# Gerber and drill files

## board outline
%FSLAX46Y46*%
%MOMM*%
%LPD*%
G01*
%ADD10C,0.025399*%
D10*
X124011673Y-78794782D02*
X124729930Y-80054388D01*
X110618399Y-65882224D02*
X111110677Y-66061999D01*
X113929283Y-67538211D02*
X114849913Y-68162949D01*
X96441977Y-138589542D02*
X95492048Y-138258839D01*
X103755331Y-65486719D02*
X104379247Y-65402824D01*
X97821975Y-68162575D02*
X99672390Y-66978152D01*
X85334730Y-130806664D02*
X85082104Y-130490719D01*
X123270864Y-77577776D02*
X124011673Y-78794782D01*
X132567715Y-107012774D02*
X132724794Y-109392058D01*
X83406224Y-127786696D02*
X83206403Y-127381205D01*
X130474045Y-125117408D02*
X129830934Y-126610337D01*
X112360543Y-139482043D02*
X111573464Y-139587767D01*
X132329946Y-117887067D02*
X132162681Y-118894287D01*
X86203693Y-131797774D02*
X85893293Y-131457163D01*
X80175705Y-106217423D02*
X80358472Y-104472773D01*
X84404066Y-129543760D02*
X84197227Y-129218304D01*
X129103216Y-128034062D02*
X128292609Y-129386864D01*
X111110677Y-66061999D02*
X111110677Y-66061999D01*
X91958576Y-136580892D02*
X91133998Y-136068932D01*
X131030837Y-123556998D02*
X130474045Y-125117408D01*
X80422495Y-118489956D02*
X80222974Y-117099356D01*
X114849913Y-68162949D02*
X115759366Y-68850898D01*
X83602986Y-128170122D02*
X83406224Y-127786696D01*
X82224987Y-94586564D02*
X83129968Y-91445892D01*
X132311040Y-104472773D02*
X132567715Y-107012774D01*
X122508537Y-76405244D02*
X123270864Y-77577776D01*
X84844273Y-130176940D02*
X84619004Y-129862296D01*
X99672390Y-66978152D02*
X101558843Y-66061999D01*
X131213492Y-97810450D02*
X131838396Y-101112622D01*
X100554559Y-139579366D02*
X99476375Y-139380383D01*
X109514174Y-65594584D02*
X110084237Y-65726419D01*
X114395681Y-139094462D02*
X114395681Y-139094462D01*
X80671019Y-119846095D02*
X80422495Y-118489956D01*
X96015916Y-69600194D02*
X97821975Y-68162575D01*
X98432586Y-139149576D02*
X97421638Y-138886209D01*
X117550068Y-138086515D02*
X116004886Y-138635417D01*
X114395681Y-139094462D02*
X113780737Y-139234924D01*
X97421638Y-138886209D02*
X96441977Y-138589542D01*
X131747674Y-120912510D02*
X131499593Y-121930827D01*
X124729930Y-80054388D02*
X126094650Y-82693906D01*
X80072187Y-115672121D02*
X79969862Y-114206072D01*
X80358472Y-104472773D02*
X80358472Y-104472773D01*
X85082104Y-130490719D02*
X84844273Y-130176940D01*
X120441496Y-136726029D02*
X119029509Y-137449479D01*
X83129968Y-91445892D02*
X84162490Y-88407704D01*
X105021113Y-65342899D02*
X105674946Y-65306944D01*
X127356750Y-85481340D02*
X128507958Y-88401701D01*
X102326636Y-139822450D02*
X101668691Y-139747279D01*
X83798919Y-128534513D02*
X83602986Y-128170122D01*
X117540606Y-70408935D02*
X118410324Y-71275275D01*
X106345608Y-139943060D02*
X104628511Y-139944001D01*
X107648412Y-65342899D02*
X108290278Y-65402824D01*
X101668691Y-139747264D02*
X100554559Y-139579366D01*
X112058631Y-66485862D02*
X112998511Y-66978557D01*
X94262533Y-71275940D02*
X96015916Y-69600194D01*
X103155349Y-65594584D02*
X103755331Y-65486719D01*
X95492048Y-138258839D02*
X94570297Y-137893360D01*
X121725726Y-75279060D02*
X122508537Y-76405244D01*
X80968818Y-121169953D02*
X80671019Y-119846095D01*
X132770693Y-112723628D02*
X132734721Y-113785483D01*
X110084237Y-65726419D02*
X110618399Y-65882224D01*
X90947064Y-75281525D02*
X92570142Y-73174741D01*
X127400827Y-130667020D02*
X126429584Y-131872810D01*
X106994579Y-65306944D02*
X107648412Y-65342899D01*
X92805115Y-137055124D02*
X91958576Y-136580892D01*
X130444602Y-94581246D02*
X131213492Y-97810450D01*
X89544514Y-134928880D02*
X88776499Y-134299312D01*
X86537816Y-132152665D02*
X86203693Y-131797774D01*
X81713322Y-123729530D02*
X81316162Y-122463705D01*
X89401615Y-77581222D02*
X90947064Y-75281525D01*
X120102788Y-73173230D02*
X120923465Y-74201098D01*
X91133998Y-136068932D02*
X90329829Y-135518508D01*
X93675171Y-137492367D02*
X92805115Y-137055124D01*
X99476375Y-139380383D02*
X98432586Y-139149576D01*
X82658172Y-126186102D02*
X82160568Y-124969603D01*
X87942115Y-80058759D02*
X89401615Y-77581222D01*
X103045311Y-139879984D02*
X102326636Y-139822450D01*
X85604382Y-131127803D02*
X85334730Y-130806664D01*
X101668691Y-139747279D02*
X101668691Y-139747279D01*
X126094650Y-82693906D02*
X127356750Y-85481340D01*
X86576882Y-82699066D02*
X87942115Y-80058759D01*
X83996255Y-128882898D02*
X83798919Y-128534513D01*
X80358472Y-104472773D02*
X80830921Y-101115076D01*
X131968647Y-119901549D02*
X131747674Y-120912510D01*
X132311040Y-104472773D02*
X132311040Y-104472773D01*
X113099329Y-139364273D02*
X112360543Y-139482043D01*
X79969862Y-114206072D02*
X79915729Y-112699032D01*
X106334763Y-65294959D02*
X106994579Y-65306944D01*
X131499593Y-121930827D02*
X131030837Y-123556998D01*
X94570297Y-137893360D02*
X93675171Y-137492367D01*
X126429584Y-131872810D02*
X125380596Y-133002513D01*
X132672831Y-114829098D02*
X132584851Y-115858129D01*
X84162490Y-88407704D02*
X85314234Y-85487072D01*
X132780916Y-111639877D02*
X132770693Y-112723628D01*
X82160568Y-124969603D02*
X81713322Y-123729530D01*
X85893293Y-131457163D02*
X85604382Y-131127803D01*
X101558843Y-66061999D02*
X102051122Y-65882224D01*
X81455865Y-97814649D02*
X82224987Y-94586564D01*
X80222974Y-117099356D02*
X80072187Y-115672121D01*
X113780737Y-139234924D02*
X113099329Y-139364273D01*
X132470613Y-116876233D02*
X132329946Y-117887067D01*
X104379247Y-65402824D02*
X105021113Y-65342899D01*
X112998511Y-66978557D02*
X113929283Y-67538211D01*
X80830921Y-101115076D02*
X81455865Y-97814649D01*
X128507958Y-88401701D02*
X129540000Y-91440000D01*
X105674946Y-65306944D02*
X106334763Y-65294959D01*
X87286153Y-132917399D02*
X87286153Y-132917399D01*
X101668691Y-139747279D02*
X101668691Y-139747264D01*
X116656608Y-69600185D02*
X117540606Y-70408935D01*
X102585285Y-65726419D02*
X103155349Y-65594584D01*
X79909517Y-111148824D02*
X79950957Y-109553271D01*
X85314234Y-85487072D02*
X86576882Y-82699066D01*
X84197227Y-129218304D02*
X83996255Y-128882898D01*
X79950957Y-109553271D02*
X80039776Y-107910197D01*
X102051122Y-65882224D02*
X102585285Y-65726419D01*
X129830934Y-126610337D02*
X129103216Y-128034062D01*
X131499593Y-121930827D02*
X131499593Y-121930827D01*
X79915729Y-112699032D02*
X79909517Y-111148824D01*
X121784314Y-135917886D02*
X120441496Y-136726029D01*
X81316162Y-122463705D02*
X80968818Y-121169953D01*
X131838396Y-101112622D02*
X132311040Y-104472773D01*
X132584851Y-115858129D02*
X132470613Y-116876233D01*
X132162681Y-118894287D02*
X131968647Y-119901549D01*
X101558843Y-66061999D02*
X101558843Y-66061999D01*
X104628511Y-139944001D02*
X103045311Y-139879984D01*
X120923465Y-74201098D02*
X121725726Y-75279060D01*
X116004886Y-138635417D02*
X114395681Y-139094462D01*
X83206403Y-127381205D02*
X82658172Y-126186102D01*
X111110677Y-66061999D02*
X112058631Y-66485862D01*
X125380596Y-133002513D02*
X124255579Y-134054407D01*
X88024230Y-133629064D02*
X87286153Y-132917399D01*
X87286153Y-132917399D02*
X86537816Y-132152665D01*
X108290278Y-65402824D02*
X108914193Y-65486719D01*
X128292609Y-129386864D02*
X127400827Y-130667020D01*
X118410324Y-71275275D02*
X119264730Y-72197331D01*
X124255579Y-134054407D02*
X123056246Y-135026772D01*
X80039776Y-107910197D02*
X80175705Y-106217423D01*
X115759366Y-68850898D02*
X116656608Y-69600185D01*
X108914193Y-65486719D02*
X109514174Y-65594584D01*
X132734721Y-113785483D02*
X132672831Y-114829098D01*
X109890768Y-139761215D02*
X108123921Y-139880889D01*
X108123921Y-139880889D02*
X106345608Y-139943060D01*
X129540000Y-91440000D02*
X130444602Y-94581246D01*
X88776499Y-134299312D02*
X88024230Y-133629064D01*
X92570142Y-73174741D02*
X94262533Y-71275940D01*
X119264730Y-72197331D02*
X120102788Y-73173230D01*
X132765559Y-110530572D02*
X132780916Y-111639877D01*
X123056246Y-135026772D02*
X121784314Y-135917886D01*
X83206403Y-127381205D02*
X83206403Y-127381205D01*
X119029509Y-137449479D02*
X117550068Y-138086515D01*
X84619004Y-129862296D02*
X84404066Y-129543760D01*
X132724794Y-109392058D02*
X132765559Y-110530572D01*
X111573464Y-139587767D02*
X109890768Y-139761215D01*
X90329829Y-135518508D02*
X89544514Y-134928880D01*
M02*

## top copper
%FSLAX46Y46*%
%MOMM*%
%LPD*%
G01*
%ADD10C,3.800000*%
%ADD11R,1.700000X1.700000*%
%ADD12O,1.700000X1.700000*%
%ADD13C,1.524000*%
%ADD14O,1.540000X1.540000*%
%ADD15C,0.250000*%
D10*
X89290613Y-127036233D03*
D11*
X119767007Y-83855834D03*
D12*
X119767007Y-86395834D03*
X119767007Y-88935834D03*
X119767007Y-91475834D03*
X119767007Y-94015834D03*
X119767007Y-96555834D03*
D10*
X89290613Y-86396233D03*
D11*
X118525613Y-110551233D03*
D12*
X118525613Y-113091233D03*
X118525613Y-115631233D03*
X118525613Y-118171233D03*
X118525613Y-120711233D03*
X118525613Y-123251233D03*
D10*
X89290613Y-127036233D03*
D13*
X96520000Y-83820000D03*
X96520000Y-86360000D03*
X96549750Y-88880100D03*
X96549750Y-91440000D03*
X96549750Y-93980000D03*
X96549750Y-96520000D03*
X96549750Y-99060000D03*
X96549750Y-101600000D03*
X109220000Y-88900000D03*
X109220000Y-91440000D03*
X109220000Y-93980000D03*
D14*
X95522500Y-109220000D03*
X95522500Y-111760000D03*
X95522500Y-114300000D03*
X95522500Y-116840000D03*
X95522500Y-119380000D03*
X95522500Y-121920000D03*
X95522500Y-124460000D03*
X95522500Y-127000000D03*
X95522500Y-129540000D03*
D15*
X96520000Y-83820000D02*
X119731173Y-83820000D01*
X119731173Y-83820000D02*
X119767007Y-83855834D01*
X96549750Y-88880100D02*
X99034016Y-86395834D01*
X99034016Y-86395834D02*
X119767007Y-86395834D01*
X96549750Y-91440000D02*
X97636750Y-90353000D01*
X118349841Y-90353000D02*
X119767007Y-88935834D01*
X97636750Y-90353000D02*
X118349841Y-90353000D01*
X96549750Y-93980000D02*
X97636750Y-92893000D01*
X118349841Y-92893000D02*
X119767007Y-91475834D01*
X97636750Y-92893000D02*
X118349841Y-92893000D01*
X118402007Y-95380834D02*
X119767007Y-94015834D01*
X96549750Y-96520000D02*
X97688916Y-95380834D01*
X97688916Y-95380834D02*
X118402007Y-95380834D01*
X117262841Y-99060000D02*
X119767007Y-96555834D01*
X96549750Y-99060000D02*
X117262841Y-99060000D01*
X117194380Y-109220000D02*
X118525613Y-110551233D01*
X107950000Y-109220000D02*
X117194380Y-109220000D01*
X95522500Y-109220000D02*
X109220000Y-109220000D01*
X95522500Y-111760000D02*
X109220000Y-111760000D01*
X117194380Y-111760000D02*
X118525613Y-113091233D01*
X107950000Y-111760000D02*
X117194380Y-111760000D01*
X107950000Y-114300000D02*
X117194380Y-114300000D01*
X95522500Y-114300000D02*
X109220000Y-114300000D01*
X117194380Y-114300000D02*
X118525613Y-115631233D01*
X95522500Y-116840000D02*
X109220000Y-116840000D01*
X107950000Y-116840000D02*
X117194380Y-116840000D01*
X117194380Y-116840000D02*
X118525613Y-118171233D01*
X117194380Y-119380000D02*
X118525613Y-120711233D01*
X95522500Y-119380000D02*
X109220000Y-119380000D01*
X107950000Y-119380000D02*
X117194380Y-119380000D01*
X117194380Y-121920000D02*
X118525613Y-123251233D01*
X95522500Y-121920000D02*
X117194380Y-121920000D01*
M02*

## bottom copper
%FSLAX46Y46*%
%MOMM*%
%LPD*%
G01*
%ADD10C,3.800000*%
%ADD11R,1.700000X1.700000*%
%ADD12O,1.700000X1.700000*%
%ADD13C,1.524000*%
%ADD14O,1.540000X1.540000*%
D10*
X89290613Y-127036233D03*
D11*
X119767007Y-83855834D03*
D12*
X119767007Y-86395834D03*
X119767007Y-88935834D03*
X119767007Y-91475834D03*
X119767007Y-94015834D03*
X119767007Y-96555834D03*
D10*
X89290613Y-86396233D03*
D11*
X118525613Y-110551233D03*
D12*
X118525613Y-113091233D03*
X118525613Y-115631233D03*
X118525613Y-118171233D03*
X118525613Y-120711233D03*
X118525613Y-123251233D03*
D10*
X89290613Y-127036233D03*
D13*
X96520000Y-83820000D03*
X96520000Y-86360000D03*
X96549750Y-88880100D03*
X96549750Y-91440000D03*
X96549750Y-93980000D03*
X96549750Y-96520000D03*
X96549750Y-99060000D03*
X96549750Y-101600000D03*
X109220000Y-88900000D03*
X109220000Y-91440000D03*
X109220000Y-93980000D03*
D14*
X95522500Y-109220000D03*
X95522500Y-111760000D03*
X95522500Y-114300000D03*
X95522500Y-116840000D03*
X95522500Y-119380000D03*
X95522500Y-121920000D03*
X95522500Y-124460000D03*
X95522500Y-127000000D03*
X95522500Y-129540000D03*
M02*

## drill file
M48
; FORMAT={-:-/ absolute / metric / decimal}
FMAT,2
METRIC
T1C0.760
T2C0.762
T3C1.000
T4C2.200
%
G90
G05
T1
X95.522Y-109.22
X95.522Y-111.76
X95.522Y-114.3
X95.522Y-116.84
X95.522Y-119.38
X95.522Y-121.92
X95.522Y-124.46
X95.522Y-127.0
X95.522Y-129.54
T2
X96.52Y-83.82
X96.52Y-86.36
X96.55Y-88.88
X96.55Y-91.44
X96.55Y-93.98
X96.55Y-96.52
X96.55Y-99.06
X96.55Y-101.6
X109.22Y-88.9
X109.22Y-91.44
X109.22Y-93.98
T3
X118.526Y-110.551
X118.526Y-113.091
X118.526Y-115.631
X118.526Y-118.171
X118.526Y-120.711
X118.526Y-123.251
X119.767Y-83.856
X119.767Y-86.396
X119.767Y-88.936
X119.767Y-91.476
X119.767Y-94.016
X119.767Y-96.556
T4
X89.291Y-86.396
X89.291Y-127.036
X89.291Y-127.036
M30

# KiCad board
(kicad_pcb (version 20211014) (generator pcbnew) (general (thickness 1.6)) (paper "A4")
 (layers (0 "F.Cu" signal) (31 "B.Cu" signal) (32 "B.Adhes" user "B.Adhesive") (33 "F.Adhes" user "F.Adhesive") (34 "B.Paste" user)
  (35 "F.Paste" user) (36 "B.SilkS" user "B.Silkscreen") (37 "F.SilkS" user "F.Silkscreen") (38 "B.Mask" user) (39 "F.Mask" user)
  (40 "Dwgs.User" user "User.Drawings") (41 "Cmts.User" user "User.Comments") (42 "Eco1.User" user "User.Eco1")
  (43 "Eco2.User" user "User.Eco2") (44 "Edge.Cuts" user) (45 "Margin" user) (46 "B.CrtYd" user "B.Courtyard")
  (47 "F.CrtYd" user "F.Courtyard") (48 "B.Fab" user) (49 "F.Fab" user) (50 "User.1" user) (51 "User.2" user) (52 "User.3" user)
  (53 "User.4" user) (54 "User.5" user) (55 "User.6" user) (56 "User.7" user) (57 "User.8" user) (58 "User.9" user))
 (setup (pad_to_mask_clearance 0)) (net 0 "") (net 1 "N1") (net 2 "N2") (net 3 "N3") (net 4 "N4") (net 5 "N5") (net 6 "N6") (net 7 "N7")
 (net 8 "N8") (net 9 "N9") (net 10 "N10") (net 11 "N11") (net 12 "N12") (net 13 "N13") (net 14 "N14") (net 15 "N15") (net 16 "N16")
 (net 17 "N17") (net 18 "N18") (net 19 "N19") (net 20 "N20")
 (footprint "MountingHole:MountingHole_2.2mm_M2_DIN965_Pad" (layer "F.Cu") (at 89.290613 127.036233)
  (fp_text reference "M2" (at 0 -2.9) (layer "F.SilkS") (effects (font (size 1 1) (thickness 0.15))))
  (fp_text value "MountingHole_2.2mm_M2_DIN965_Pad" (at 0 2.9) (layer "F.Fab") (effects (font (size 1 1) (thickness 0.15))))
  (pad "1" thru_hole circle (at 0 0) (size 3.8 3.8) (drill 2.2) (layers *.Cu *.Mask)))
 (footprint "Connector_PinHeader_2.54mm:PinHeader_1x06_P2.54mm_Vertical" (layer "F.Cu") (at 119.767007 83.855834)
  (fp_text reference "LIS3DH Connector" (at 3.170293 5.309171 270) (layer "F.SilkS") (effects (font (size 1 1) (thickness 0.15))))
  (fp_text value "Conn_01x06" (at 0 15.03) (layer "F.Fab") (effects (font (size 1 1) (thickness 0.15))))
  (pad "1" thru_hole rect (at 0 0) (size 1.7 1.7) (drill 1) (layers *.Cu *.Mask) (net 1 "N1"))
  (pad "2" thru_hole oval (at 0 2.54) (size 1.7 1.7) (drill 1) (layers *.Cu *.Mask) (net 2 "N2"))
  (pad "3" thru_hole oval (at 0 5.08) (size 1.7 1.7) (drill 1) (layers *.Cu *.Mask) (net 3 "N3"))
  (pad "4" thru_hole oval (at 0 7.62) (size 1.7 1.7) (drill 1) (layers *.Cu *.Mask) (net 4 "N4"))
  (pad "5" thru_hole oval (at 0 10.16) (size 1.7 1.7) (drill 1) (layers *.Cu *.Mask) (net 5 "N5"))
  (pad "6" thru_hole oval (at 0 12.7) (size 1.7 1.7) (drill 1) (layers *.Cu *.Mask) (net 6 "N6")))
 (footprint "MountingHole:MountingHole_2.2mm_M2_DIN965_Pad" (layer "F.Cu") (at 89.290613 86.396233)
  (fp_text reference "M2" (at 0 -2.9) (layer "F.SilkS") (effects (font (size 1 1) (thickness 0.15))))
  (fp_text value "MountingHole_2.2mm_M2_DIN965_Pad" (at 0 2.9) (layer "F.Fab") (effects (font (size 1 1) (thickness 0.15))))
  (pad "1" thru_hole circle (at 0 0) (size 3.8 3.8) (drill 2.2) (layers *.Cu *.Mask)))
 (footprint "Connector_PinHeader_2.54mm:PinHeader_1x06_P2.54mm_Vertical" (layer "F.Cu") (at 118.525613 110.551233)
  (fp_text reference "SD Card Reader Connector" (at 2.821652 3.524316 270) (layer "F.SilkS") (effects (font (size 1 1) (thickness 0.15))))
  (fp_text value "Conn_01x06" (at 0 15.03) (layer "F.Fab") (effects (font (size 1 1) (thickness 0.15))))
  (pad "1" thru_hole rect (at 0 0) (size 1.7 1.7) (drill 1) (layers *.Cu *.Mask) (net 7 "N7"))
  (pad "2" thru_hole oval (at 0 2.54) (size 1.7 1.7) (drill 1) (layers *.Cu *.Mask) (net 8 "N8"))
  (pad "3" thru_hole oval (at 0 5.08) (size 1.7 1.7) (drill 1) (layers *.Cu *.Mask) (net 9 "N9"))
  (pad "4" thru_hole oval (at 0 7.62) (size 1.7 1.7) (drill 1) (layers *.Cu *.Mask) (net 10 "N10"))
  (pad "5" thru_hole oval (at 0 10.16) (size 1.7 1.7) (drill 1) (layers *.Cu *.Mask) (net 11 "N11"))
  (pad "6" thru_hole oval (at 0 12.7) (size 1.7 1.7) (drill 1) (layers *.Cu *.Mask) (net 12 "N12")))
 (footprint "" (layer "F.Cu") (at 89.290613 127.036233)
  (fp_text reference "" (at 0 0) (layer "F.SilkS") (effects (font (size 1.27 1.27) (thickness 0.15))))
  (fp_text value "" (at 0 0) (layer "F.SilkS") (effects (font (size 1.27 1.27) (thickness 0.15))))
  (pad "1" thru_hole circle (at 0 0) (size 3.8 3.8) (drill 2.2) (layers *.Cu *.Mask)))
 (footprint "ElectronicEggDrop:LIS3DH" (layer "B.Cu") (at 104.14 78.74 180)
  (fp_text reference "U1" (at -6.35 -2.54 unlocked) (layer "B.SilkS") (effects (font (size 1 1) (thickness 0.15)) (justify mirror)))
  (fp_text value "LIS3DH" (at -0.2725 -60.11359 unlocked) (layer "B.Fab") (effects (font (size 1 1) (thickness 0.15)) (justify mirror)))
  (pad "1" thru_hole circle (at 7.62 -5.08 180) (size 1.524 1.524) (drill 0.762) (layers *.Cu *.Mask) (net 1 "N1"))
  (pad "2" thru_hole circle (at 7.62 -7.62 180) (size 1.524 1.524) (drill 0.762) (layers *.Cu *.Mask) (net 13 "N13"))
  (pad "3" thru_hole circle (at 7.59025 -10.1401 180) (size 1.524 1.524) (drill 0.762) (layers *.Cu *.Mask) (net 2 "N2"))
  (pad "4" thru_hole circle (at 7.59025 -12.7 180) (size 1.524 1.524) (drill 0.762) (layers *.Cu *.Mask) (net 3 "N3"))
  (pad "5" thru_hole circle (at 7.59025 -15.24 180) (size 1.524 1.524) (drill 0.762) (layers *.Cu *.Mask) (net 4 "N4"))
  (pad "6" thru_hole circle (at 7.59025 -17.78 180) (size 1.524 1.524) (drill 0.762) (layers *.Cu *.Mask) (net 5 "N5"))
  (pad "7" thru_hole circle (at 7.59025 -20.32 180) (size 1.524 1.524) (drill 0.762) (layers *.Cu *.Mask) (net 6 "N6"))
  (pad "8" thru_hole circle (at 7.59025 -22.86 180) (size 1.524 1.524) (drill 0.762) (layers *.Cu *.Mask) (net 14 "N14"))
  (pad "9" thru_hole circle (at -5.08 -10.16 180) (size 1.524 1.524) (drill 0.762) (layers *.Cu *.Mask) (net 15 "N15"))
  (pad "10" thru_hole circle (at -5.08 -12.7 180) (size 1.524 1.524) (drill 0.762) (layers *.Cu *.Mask) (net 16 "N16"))
  (pad "11" thru_hole circle (at -5.08 -15.24 180) (size 1.524 1.524) (drill 0.762) (layers *.Cu *.Mask) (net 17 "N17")))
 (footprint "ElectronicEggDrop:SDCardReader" (layer "B.Cu") (at 94.2525 119.38 -90)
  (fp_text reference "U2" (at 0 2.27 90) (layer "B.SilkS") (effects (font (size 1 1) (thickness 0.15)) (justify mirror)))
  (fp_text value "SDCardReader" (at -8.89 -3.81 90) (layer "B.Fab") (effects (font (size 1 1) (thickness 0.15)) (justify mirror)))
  (pad "1" thru_hole oval (at -10.16 -1.27 270) (size 1.54 1.54) (drill 0.76) (layers *.Cu *.Mask) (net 7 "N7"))
  (pad "2" thru_hole oval (at -7.62 -1.27 270) (size 1.54 1.54) (drill 0.76) (layers *.Cu *.Mask) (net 8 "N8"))
  (pad "3" thru_hole oval (at -5.08 -1.27 270) (size 1.54 1.54) (drill 0.76) (layers *.Cu *.Mask) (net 9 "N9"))
  (pad "4" thru_hole oval (at -2.54 -1.27 270) (size 1.54 1.54) (drill 0.76) (layers *.Cu *.Mask) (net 10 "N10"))
  (pad "5" thru_hole oval (at 0 -1.27 270) (size 1.54 1.54) (drill 0.76) (layers *.Cu *.Mask) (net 11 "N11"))
  (pad "6" thru_hole oval (at 2.54 -1.27 270) (size 1.54 1.54) (drill 0.76) (layers *.Cu *.Mask) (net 12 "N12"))
  (pad "7" thru_hole oval (at 5.08 -1.27 270) (size 1.54 1.54) (drill 0.76) (layers *.Cu *.Mask) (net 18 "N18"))
  (pad "8" thru_hole oval (at 7.62 -1.27 270) (size 1.54 1.54) (drill 0.76) (layers *.Cu *.Mask) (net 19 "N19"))
  (pad "9" thru_hole oval (at 10.16 -1.27 270) (size 1.54 1.54) (drill 0.76) (layers *.Cu *.Mask) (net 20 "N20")))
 (gr_line (start 124.011673 78.794782) (end 124.72993 80.054388) (layer "Edge.Cuts") (width 0.025399))
 (gr_line (start 110.618399 65.882224) (end 111.110677 66.061999) (layer "Edge.Cuts") (width 0.025399))
 (gr_line (start 113.929283 67.538211) (end 114.849913 68.162949) (layer "Edge.Cuts") (width 0.025399))
 (gr_line (start 96.441977 138.589542) (end 95.492048 138.258839) (layer "Edge.Cuts") (width 0.025399))
 (gr_line (start 103.755331 65.486719) (end 104.379247 65.402824) (layer "Edge.Cuts") (width 0.025399))
 (gr_line (start 97.821975 68.162575) (end 99.67239 66.978152) (layer "Edge.Cuts") (width 0.025399))
 (gr_line (start 85.33473 130.806664) (end 85.082104 130.490719) (layer "Edge.Cuts") (width 0.025399))
 (gr_line (start 123.270864 77.577776) (end 124.011673 78.794782) (layer "Edge.Cuts") (width 0.025399))
 (gr_line (start 132.567715 107.012774) (end 132.724794 109.392058) (layer "Edge.Cuts") (width 0.025399))
 (gr_line (start 83.406224 127.786696) (end 83.206403 127.381205) (layer "Edge.Cuts") (width 0.025399))
 (gr_line (start 130.474045 125.117408) (end 129.830934 126.610337) (layer "Edge.Cuts") (width 0.025399))
 (gr_line (start 112.360543 139.482043) (end 111.573464 139.587767) (layer "Edge.Cuts") (width 0.025399))
 (gr_line (start 132.329946 117.887067) (end 132.162681 118.894287) (layer "Edge.Cuts") (width 0.025399))
 (gr_line (start 86.203693 131.797774) (end 85.893293 131.457163) (layer "Edge.Cuts") (width 0.025399))
 (gr_line (start 80.175705 106.217423) (end 80.358472 104.472773) (layer "Edge.Cuts") (width 0.025399))
 (gr_line (start 84.404066 129.54376) (end 84.197227 129.218304) (layer "Edge.Cuts") (width 0.025399))
 (gr_line (start 129.103216 128.034062) (end 128.292609 129.386864) (layer "Edge.Cuts") (width 0.025399))
 (gr_line (start 111.110677 66.061999) (end 111.110677 66.061999) (layer "Edge.Cuts") (width 0.025399))
 (gr_line (start 91.958576 136.580892) (end 91.133998 136.068932) (layer "Edge.Cuts") (width 0.025399))
 (gr_line (start 131.030837 123.556998) (end 130.474045 125.117408) (layer "Edge.Cuts") (width 0.025399))
 (gr_line (start 80.422495 118.489956) (end 80.222974 117.099356) (layer "Edge.Cuts") (width 0.025399))
 (gr_line (start 114.849913 68.162949) (end 115.759366 68.850898) (layer "Edge.Cuts") (width 0.025399))
 (gr_line (start 83.602986 128.170122) (end 83.406224 127.786696) (layer "Edge.Cuts") (width 0.025399))
 (gr_line (start 82.224987 94.586564) (end 83.129968 91.445892) (layer "Edge.Cuts") (width 0.025399))
 (gr_line (start 132.31104 104.472773) (end 132.567715 107.012774) (layer "Edge.Cuts") (width 0.025399))
 (gr_line (start 122.508537 76.405244) (end 123.270864 77.577776) (layer "Edge.Cuts") (width 0.025399))
 (gr_line (start 84.844273 130.17694) (end 84.619004 129.862296) (layer "Edge.Cuts") (width 0.025399))
 (gr_line (start 99.67239 66.978152) (end 101.558843 66.061999) (layer "Edge.Cuts") (width 0.025399))
 (gr_line (start 131.213492 97.81045) (end 131.838396 101.112622) (layer "Edge.Cuts") (width 0.025399))
 (gr_line (start 100.554559 139.579366) (end 99.476375 139.380383) (layer "Edge.Cuts") (width 0.025399))
 (gr_line (start 109.514174 65.594584) (end 110.084237 65.726419) (layer "Edge.Cuts") (width 0.025399))
 (gr_line (start 114.395681 139.094462) (end 114.395681 139.094462) (layer "Edge.Cuts") (width 0.025399))
 (gr_line (start 80.671019 119.846095) (end 80.422495 118.489956) (layer "Edge.Cuts") (width 0.025399))
 (gr_line (start 96.015916 69.600194) (end 97.821975 68.162575) (layer "Edge.Cuts") (width 0.025399))
 (gr_line (start 98.432586 139.149576) (end 97.421638 138.886209) (layer "Edge.Cuts") (width 0.025399))
 (gr_line (start 117.550068 138.086515) (end 116.004886 138.635417) (layer "Edge.Cuts") (width 0.025399))
 (gr_line (start 114.395681 139.094462) (end 113.780737 139.234924) (layer "Edge.Cuts") (width 0.025399))
 (gr_line (start 97.421638 138.886209) (end 96.441977 138.589542) (layer "Edge.Cuts") (width 0.025399))
 (gr_line (start 131.747674 120.91251) (end 131.499593 121.930827) (layer "Edge.Cuts") (width 0.025399))
 (gr_line (start 124.72993 80.054388) (end 126.09465 82.693906) (layer "Edge.Cuts") (width 0.025399))
 (gr_line (start 80.072187 115.672121) (end 79.969862 114.206072) (layer "Edge.Cuts") (width 0.025399))
 (gr_line (start 80.358472 104.472773) (end 80.358472 104.472773) (layer "Edge.Cuts") (width 0.025399))
 (gr_line (start 85.082104 130.490719) (end 84.844273 130.17694) (layer "Edge.Cuts") (width 0.025399))
 (gr_line (start 120.441496 136.726029) (end 119.029509 137.449479) (layer "Edge.Cuts") (width 0.025399))
 (gr_line (start 83.129968 91.445892) (end 84.16249 88.407704) (layer "Edge.Cuts") (width 0.025399))
 (gr_line (start 105.021113 65.342899) (end 105.674946 65.306944) (layer "Edge.Cuts") (width 0.025399))
 (gr_line (start 127.35675 85.48134) (end 128.507958 88.401701) (layer "Edge.Cuts") (width 0.025399))
 (gr_line (start 102.326636 139.82245) (end 101.668691 139.747279) (layer "Edge.Cuts") (width 0.025399))
 (gr_line (start 83.798919 128.534513) (end 83.602986 128.170122) (layer "Edge.Cuts") (width 0.025399))
 (gr_line (start 117.540606 70.408935) (end 118.410324 71.275275) (layer "Edge.Cuts") (width 0.025399))
 (gr_line (start 106.345608 139.94306) (end 104.628511 139.944001) (layer "Edge.Cuts") (width 0.025399))
 (gr_line (start 107.648412 65.342899) (end 108.290278 65.402824) (layer "Edge.Cuts") (width 0.025399))
 (gr_line (start 101.668691 139.747264) (end 100.554559 139.579366) (layer "Edge.Cuts") (width 0.025399))
 (gr_line (start 112.058631 66.485862) (end 112.998511 66.978557) (layer "Edge.Cuts") (width 0.025399))
 (gr_line (start 94.262533 71.27594) (end 96.015916 69.600194) (layer "Edge.Cuts") (width 0.025399))
 (gr_line (start 103.155349 65.594584) (end 103.755331 65.486719) (layer "Edge.Cuts") (width 0.025399))
 (gr_line (start 95.492048 138.258839) (end 94.570297 137.89336) (layer "Edge.Cuts") (width 0.025399))
 (gr_line (start 121.725726 75.27906) (end 122.508537 76.405244) (layer "Edge.Cuts") (width 0.025399))
 (gr_line (start 80.968818 121.169953) (end 80.671019 119.846095) (layer "Edge.Cuts") (width 0.025399))
 (gr_line (start 132.770693 112.723628) (end 132.734721 113.785483) (layer "Edge.Cuts") (width 0.025399))
 (gr_line (start 110.084237 65.726419) (end 110.618399 65.882224) (layer "Edge.Cuts") (width 0.025399))
 (gr_line (start 90.947064 75.281525) (end 92.570142 73.174741) (layer "Edge.Cuts") (width 0.025399))
 (gr_line (start 127.400827 130.66702) (end 126.429584 131.87281) (layer "Edge.Cuts") (width 0.025399))
 (gr_line (start 106.994579 65.306944) (end 107.648412 65.342899) (layer "Edge.Cuts") (width 0.025399))
 (gr_line (start 92.805115 137.055124) (end 91.958576 136.580892) (layer "Edge.Cuts") (width 0.025399))
 (gr_line (start 130.444602 94.581246) (end 131.213492 97.81045) (layer "Edge.Cuts") (width 0.025399))
 (gr_line (start 89.544514 134.92888) (end 88.776499 134.299312) (layer "Edge.Cuts") (width 0.025399))
 (gr_line (start 86.537816 132.152665) (end 86.203693 131.797774) (layer "Edge.Cuts") (width 0.025399))
 (gr_line (start 81.713322 123.72953) (end 81.316162 122.463705) (layer "Edge.Cuts") (width 0.025399))
 (gr_line (start 89.401615 77.581222) (end 90.947064 75.281525) (layer "Edge.Cuts") (width 0.025399))
 (gr_line (start 120.102788 73.17323) (end 120.923465 74.201098) (layer "Edge.Cuts") (width 0.025399))
 (gr_line (start 91.133998 136.068932) (end 90.329829 135.518508) (layer "Edge.Cuts") (width 0.025399))
 (gr_line (start 93.675171 137.492367) (end 92.805115 137.055124) (layer "Edge.Cuts") (width 0.025399))
 (gr_line (start 99.476375 139.380383) (end 98.432586 139.149576) (layer "Edge.Cuts") (width 0.025399))
 (gr_line (start 82.658172 126.186102) (end 82.160568 124.969603) (layer "Edge.Cuts") (width 0.025399))
 (gr_line (start 87.942115 80.058759) (end 89.401615 77.581222) (layer "Edge.Cuts") (width 0.025399))
 (gr_line (start 103.045311 139.879984) (end 102.326636 139.82245) (layer "Edge.Cuts") (width 0.025399))
 (gr_line (start 85.604382 131.127803) (end 85.33473 130.806664) (layer "Edge.Cuts") (width 0.025399))
 (gr_line (start 101.668691 139.747279) (end 101.668691 139.747279) (layer "Edge.Cuts") (width 0.025399))
 (gr_line (start 126.09465 82.693906) (end 127.35675 85.48134) (layer "Edge.Cuts") (width 0.025399))
 (gr_line (start 86.576882 82.699066) (end 87.942115 80.058759) (layer "Edge.Cuts") (width 0.025399))
 (gr_line (start 83.996255 128.882898) (end 83.798919 128.534513) (layer "Edge.Cuts") (width 0.025399))
 (gr_line (start 80.358472 104.472773) (end 80.830921 101.115076) (layer "Edge.Cuts") (width 0.025399))
 (gr_line (start 131.968647 119.901549) (end 131.747674 120.91251) (layer "Edge.Cuts") (width 0.025399))
 (gr_line (start 132.31104 104.472773) (end 132.31104 104.472773) (layer "Edge.Cuts") (width 0.025399))
 (gr_line (start 113.099329 139.364273) (end 112.360543 139.482043) (layer "Edge.Cuts") (width 0.025399))
 (gr_line (start 79.969862 114.206072) (end 79.915729 112.699032) (layer "Edge.Cuts") (width 0.025399))
 (gr_line (start 106.334763 65.294959) (end 106.994579 65.306944) (layer "Edge.Cuts") (width 0.025399))
 (gr_line (start 131.499593 121.930827) (end 131.030837 123.556998) (layer "Edge.Cuts") (width 0.025399))
 (gr_line (start 94.570297 137.89336) (end 93.675171 137.492367) (layer "Edge.Cuts") (width 0.025399))
 (gr_line (start 126.429584 131.87281) (end 125.380596 133.002513) (layer "Edge.Cuts") (width 0.025399))
 (gr_line (start 132.672831 114.829098) (end 132.584851 115.858129) (layer "Edge.Cuts") (width 0.025399))
 (gr_line (start 84.16249 88.407704) (end 85.314234 85.487072) (layer "Edge.Cuts") (width 0.025399))
 (gr_line (start 132.780916 111.639877) (end 132.770693 112.723628) (layer "Edge.Cuts") (width 0.025399))
 (gr_line (start 82.160568 124.969603) (end 81.713322 123.72953) (layer "Edge.Cuts") (width 0.025399))
 (gr_line (start 85.893293 131.457163) (end 85.604382 131.127803) (layer "Edge.Cuts") (width 0.025399))
 (gr_line (start 101.558843 66.061999) (end 102.051122 65.882224) (layer "Edge.Cuts") (width 0.025399))
 (gr_line (start 81.455865 97.814649) (end 82.224987 94.586564) (layer "Edge.Cuts") (width 0.025399))
 (gr_line (start 80.222974 117.099356) (end 80.072187 115.672121) (layer "Edge.Cuts") (width 0.025399))
 (gr_line (start 113.780737 139.234924) (end 113.099329 139.364273) (layer "Edge.Cuts") (width 0.025399))
 (gr_line (start 132.470613 116.876233) (end 132.329946 117.887067) (layer "Edge.Cuts") (width 0.025399))
 (gr_line (start 104.379247 65.402824) (end 105.021113 65.342899) (layer "Edge.Cuts") (width 0.025399))
 (gr_line (start 112.998511 66.978557) (end 113.929283 67.538211) (layer "Edge.Cuts") (width 0.025399))
 (gr_line (start 80.830921 101.115076) (end 81.455865 97.814649) (layer "Edge.Cuts") (width 0.025399))
 (gr_line (start 128.507958 88.401701) (end 129.54 91.44) (layer "Edge.Cuts") (width 0.025399))
 (gr_line (start 105.674946 65.306944) (end 106.334763 65.294959) (layer "Edge.Cuts") (width 0.025399))
 (gr_line (start 87.286153 132.917399) (end 87.286153 132.917399) (layer "Edge.Cuts") (width 0.025399))
 (gr_line (start 101.668691 139.747279) (end 101.668691 139.747264) (layer "Edge.Cuts") (width 0.025399))
 (gr_line (start 116.656608 69.600185) (end 117.540606 70.408935) (layer "Edge.Cuts") (width 0.025399))
 (gr_line (start 102.585285 65.726419) (end 103.155349 65.594584) (layer "Edge.Cuts") (width 0.025399))
 (gr_line (start 79.909517 111.148824) (end 79.950957 109.553271) (layer "Edge.Cuts") (width 0.025399))
 (gr_line (start 85.314234 85.487072) (end 86.576882 82.699066) (layer "Edge.Cuts") (width 0.025399))
 (gr_line (start 84.197227 129.218304) (end 83.996255 128.882898) (layer "Edge.Cuts") (width 0.025399))
 (gr_line (start 79.950957 109.553271) (end 80.039776 107.910197) (layer "Edge.Cuts") (width 0.025399))
 (gr_line (start 102.051122 65.882224) (end 102.585285 65.726419) (layer "Edge.Cuts") (width 0.025399))
 (gr_line (start 129.830934 126.610337) (end 129.103216 128.034062) (layer "Edge.Cuts") (width 0.025399))
 (gr_line (start 131.499593 121.930827) (end 131.499593 121.930827) (layer "Edge.Cuts") (width 0.025399))
 (gr_line (start 79.915729 112.699032) (end 79.909517 111.148824) (layer "Edge.Cuts") (width 0.025399))
 (gr_line (start 121.784314 135.917886) (end 120.441496 136.726029) (layer "Edge.Cuts") (width 0.025399))
 (gr_line (start 81.316162 122.463705) (end 80.968818 121.169953) (layer "Edge.Cuts") (width 0.025399))
 (gr_line (start 131.838396 101.112622) (end 132.31104 104.472773) (layer "Edge.Cuts") (width 0.025399))
 (gr_line (start 132.584851 115.858129) (end 132.470613 116.876233) (layer "Edge.Cuts") (width 0.025399))
 (gr_line (start 132.162681 118.894287) (end 131.968647 119.901549) (layer "Edge.Cuts") (width 0.025399))
 (gr_line (start 101.558843 66.061999) (end 101.558843 66.061999) (layer "Edge.Cuts") (width 0.025399))
 (gr_line (start 104.628511 139.944001) (end 103.045311 139.879984) (layer "Edge.Cuts") (width 0.025399))
 (gr_line (start 120.923465 74.201098) (end 121.725726 75.27906) (layer "Edge.Cuts") (width 0.025399))
 (gr_line (start 116.004886 138.635417) (end 114.395681 139.094462) (layer "Edge.Cuts") (width 0.025399))
 (gr_line (start 83.206403 127.381205) (end 82.658172 126.186102) (layer "Edge.Cuts") (width 0.025399))
 (gr_line (start 111.110677 66.061999) (end 112.058631 66.485862) (layer "Edge.Cuts") (width 0.025399))
 (gr_line (start 125.380596 133.002513) (end 124.255579 134.054407) (layer "Edge.Cuts") (width 0.025399))
 (gr_line (start 88.02423 133.629064) (end 87.286153 132.917399) (layer "Edge.Cuts") (width 0.025399))
 (gr_line (start 87.286153 132.917399) (end 86.537816 132.152665) (layer "Edge.Cuts") (width 0.025399))
 (gr_line (start 108.290278 65.402824) (end 108.914193 65.486719) (layer "Edge.Cuts") (width 0.025399))
 (gr_line (start 128.292609 129.386864) (end 127.400827 130.66702) (layer "Edge.Cuts") (width 0.025399))
 (gr_line (start 118.410324 71.275275) (end 119.26473 72.197331) (layer "Edge.Cuts") (width 0.025399))
 (gr_line (start 124.255579 134.054407) (end 123.056246 135.026772) (layer "Edge.Cuts") (width 0.025399))
 (gr_line (start 80.039776 107.910197) (end 80.175705 106.217423) (layer "Edge.Cuts") (width 0.025399))
 (gr_line (start 115.759366 68.850898) (end 116.656608 69.600185) (layer "Edge.Cuts") (width 0.025399))
 (gr_line (start 108.914193 65.486719) (end 109.514174 65.594584) (layer "Edge.Cuts") (width 0.025399))
 (gr_line (start 132.734721 113.785483) (end 132.672831 114.829098) (layer "Edge.Cuts") (width 0.025399))
 (gr_line (start 109.890768 139.761215) (end 108.123921 139.880889) (layer "Edge.Cuts") (width 0.025399))
 (gr_line (start 108.123921 139.880889) (end 106.345608 139.94306) (layer "Edge.Cuts") (width 0.025399))
 (gr_line (start 129.54 91.44) (end 130.444602 94.581246) (layer "Edge.Cuts") (width 0.025399))
 (gr_line (start 88.776499 134.299312) (end 88.02423 133.629064) (layer "Edge.Cuts") (width 0.025399))
 (gr_line (start 92.570142 73.174741) (end 94.262533 71.27594) (layer "Edge.Cuts") (width 0.025399))
 (gr_line (start 119.26473 72.197331) (end 120.102788 73.17323) (layer "Edge.Cuts") (width 0.025399))
 (gr_line (start 132.765559 110.530572) (end 132.780916 111.639877) (layer "Edge.Cuts") (width 0.025399))
 (gr_line (start 123.056246 135.026772) (end 121.784314 135.917886) (layer "Edge.Cuts") (width 0.025399))
 (gr_line (start 83.206403 127.381205) (end 83.206403 127.381205) (layer "Edge.Cuts") (width 0.025399))
 (gr_line (start 119.029509 137.449479) (end 117.550068 138.086515) (layer "Edge.Cuts") (width 0.025399))
 (gr_line (start 84.619004 129.862296) (end 84.404066 129.54376) (layer "Edge.Cuts") (width 0.025399))
 (gr_line (start 132.724794 109.392058) (end 132.765559 110.530572) (layer "Edge.Cuts") (width 0.025399))
 (gr_line (start 111.573464 139.587767) (end 109.890768 139.761215) (layer "Edge.Cuts") (width 0.025399))
 (gr_line (start 90.329829 135.518508) (end 89.544514 134.92888) (layer "Edge.Cuts") (width 0.025399))
 (segment (start 96.52 83.82) (end 119.731173 83.82) (width 0.25) (layer "F.Cu") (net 1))
 (segment (start 119.731173 83.82) (end 119.767007 83.855834) (width 0.25) (layer "F.Cu") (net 1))
 (segment (start 96.54975 88.8801) (end 99.034016 86.395834) (width 0.25) (layer "F.Cu") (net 2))
 (segment (start 99.034016 86.395834) (end 119.767007 86.395834) (width 0.25) (layer "F.Cu") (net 2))
 (segment (start 96.54975 91.44) (end 97.63675 90.353) (width 0.25) (layer "F.Cu") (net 3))
 (segment (start 118.349841 90.353) (end 119.767007 88.935834) (width 0.25) (layer "F.Cu") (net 3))
 (segment (start 97.63675 90.353) (end 118.349841 90.353) (width 0.25) (layer "F.Cu") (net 3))
 (segment (start 96.54975 93.98) (end 97.63675 92.893) (width 0.25) (layer "F.Cu") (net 4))
 (segment (start 118.349841 92.893) (end 119.767007 91.475834) (width 0.25) (layer "F.Cu") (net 4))
 (segment (start 97.63675 92.893) (end 118.349841 92.893) (width 0.25) (layer "F.Cu") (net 4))
 (segment (start 118.402007 95.380834) (end 119.767007 94.015834) (width 0.25) (layer "F.Cu") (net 5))
 (segment (start 96.54975 96.52) (end 97.688916 95.380834) (width 0.25) (layer "F.Cu") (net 5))
 (segment (start 97.688916 95.380834) (end 118.402007 95.380834) (width 0.25) (layer "F.Cu") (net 5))
 (segment (start 117.262841 99.06) (end 119.767007 96.555834) (width 0.25) (layer "F.Cu") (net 6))
 (segment (start 96.54975 99.06) (end 117.262841 99.06) (width 0.25) (layer "F.Cu") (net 6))
 (segment (start 117.19438 109.22) (end 118.525613 110.551233) (width 0.25) (layer "F.Cu") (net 7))
 (segment (start 107.95 109.22) (end 117.19438 109.22) (width 0.25) (layer "F.Cu") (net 7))
 (segment (start 95.5225 109.22) (end 109.22 109.22) (width 0.25) (layer "F.Cu") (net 7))
 (segment (start 95.5225 111.76) (end 109.22 111.76) (width 0.25) (layer "F.Cu") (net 8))
 (segment (start 117.19438 111.76) (end 118.525613 113.091233) (width 0.25) (layer "F.Cu") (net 8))
 (segment (start 107.95 111.76) (end 117.19438 111.76) (width 0.25) (layer "F.Cu") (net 8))
 (segment (start 107.95 114.3) (end 117.19438 114.3) (width 0.25) (layer "F.Cu") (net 9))
 (segment (start 95.5225 114.3) (end 109.22 114.3) (width 0.25) (layer "F.Cu") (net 9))
 (segment (start 117.19438 114.3) (end 118.525613 115.631233) (width 0.25) (layer "F.Cu") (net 9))
 (segment (start 95.5225 116.84) (end 109.22 116.84) (width 0.25) (layer "F.Cu") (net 10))
 (segment (start 107.95 116.84) (end 117.19438 116.84) (width 0.25) (layer "F.Cu") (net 10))
 (segment (start 117.19438 116.84) (end 118.525613 118.171233) (width 0.25) (layer "F.Cu") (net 10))
 (segment (start 117.19438 119.38) (end 118.525613 120.711233) (width 0.25) (layer "F.Cu") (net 11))
 (segment (start 95.5225 119.38) (end 109.22 119.38) (width 0.25) (layer "F.Cu") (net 11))
 (segment (start 107.95 119.38) (end 117.19438 119.38) (width 0.25) (layer "F.Cu") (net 11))
 (segment (start 117.19438 121.92) (end 118.525613 123.251233) (width 0.25) (layer "F.Cu") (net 12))
 (segment (start 95.5225 121.92) (end 117.19438 121.92) (width 0.25) (layer "F.Cu") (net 12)))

